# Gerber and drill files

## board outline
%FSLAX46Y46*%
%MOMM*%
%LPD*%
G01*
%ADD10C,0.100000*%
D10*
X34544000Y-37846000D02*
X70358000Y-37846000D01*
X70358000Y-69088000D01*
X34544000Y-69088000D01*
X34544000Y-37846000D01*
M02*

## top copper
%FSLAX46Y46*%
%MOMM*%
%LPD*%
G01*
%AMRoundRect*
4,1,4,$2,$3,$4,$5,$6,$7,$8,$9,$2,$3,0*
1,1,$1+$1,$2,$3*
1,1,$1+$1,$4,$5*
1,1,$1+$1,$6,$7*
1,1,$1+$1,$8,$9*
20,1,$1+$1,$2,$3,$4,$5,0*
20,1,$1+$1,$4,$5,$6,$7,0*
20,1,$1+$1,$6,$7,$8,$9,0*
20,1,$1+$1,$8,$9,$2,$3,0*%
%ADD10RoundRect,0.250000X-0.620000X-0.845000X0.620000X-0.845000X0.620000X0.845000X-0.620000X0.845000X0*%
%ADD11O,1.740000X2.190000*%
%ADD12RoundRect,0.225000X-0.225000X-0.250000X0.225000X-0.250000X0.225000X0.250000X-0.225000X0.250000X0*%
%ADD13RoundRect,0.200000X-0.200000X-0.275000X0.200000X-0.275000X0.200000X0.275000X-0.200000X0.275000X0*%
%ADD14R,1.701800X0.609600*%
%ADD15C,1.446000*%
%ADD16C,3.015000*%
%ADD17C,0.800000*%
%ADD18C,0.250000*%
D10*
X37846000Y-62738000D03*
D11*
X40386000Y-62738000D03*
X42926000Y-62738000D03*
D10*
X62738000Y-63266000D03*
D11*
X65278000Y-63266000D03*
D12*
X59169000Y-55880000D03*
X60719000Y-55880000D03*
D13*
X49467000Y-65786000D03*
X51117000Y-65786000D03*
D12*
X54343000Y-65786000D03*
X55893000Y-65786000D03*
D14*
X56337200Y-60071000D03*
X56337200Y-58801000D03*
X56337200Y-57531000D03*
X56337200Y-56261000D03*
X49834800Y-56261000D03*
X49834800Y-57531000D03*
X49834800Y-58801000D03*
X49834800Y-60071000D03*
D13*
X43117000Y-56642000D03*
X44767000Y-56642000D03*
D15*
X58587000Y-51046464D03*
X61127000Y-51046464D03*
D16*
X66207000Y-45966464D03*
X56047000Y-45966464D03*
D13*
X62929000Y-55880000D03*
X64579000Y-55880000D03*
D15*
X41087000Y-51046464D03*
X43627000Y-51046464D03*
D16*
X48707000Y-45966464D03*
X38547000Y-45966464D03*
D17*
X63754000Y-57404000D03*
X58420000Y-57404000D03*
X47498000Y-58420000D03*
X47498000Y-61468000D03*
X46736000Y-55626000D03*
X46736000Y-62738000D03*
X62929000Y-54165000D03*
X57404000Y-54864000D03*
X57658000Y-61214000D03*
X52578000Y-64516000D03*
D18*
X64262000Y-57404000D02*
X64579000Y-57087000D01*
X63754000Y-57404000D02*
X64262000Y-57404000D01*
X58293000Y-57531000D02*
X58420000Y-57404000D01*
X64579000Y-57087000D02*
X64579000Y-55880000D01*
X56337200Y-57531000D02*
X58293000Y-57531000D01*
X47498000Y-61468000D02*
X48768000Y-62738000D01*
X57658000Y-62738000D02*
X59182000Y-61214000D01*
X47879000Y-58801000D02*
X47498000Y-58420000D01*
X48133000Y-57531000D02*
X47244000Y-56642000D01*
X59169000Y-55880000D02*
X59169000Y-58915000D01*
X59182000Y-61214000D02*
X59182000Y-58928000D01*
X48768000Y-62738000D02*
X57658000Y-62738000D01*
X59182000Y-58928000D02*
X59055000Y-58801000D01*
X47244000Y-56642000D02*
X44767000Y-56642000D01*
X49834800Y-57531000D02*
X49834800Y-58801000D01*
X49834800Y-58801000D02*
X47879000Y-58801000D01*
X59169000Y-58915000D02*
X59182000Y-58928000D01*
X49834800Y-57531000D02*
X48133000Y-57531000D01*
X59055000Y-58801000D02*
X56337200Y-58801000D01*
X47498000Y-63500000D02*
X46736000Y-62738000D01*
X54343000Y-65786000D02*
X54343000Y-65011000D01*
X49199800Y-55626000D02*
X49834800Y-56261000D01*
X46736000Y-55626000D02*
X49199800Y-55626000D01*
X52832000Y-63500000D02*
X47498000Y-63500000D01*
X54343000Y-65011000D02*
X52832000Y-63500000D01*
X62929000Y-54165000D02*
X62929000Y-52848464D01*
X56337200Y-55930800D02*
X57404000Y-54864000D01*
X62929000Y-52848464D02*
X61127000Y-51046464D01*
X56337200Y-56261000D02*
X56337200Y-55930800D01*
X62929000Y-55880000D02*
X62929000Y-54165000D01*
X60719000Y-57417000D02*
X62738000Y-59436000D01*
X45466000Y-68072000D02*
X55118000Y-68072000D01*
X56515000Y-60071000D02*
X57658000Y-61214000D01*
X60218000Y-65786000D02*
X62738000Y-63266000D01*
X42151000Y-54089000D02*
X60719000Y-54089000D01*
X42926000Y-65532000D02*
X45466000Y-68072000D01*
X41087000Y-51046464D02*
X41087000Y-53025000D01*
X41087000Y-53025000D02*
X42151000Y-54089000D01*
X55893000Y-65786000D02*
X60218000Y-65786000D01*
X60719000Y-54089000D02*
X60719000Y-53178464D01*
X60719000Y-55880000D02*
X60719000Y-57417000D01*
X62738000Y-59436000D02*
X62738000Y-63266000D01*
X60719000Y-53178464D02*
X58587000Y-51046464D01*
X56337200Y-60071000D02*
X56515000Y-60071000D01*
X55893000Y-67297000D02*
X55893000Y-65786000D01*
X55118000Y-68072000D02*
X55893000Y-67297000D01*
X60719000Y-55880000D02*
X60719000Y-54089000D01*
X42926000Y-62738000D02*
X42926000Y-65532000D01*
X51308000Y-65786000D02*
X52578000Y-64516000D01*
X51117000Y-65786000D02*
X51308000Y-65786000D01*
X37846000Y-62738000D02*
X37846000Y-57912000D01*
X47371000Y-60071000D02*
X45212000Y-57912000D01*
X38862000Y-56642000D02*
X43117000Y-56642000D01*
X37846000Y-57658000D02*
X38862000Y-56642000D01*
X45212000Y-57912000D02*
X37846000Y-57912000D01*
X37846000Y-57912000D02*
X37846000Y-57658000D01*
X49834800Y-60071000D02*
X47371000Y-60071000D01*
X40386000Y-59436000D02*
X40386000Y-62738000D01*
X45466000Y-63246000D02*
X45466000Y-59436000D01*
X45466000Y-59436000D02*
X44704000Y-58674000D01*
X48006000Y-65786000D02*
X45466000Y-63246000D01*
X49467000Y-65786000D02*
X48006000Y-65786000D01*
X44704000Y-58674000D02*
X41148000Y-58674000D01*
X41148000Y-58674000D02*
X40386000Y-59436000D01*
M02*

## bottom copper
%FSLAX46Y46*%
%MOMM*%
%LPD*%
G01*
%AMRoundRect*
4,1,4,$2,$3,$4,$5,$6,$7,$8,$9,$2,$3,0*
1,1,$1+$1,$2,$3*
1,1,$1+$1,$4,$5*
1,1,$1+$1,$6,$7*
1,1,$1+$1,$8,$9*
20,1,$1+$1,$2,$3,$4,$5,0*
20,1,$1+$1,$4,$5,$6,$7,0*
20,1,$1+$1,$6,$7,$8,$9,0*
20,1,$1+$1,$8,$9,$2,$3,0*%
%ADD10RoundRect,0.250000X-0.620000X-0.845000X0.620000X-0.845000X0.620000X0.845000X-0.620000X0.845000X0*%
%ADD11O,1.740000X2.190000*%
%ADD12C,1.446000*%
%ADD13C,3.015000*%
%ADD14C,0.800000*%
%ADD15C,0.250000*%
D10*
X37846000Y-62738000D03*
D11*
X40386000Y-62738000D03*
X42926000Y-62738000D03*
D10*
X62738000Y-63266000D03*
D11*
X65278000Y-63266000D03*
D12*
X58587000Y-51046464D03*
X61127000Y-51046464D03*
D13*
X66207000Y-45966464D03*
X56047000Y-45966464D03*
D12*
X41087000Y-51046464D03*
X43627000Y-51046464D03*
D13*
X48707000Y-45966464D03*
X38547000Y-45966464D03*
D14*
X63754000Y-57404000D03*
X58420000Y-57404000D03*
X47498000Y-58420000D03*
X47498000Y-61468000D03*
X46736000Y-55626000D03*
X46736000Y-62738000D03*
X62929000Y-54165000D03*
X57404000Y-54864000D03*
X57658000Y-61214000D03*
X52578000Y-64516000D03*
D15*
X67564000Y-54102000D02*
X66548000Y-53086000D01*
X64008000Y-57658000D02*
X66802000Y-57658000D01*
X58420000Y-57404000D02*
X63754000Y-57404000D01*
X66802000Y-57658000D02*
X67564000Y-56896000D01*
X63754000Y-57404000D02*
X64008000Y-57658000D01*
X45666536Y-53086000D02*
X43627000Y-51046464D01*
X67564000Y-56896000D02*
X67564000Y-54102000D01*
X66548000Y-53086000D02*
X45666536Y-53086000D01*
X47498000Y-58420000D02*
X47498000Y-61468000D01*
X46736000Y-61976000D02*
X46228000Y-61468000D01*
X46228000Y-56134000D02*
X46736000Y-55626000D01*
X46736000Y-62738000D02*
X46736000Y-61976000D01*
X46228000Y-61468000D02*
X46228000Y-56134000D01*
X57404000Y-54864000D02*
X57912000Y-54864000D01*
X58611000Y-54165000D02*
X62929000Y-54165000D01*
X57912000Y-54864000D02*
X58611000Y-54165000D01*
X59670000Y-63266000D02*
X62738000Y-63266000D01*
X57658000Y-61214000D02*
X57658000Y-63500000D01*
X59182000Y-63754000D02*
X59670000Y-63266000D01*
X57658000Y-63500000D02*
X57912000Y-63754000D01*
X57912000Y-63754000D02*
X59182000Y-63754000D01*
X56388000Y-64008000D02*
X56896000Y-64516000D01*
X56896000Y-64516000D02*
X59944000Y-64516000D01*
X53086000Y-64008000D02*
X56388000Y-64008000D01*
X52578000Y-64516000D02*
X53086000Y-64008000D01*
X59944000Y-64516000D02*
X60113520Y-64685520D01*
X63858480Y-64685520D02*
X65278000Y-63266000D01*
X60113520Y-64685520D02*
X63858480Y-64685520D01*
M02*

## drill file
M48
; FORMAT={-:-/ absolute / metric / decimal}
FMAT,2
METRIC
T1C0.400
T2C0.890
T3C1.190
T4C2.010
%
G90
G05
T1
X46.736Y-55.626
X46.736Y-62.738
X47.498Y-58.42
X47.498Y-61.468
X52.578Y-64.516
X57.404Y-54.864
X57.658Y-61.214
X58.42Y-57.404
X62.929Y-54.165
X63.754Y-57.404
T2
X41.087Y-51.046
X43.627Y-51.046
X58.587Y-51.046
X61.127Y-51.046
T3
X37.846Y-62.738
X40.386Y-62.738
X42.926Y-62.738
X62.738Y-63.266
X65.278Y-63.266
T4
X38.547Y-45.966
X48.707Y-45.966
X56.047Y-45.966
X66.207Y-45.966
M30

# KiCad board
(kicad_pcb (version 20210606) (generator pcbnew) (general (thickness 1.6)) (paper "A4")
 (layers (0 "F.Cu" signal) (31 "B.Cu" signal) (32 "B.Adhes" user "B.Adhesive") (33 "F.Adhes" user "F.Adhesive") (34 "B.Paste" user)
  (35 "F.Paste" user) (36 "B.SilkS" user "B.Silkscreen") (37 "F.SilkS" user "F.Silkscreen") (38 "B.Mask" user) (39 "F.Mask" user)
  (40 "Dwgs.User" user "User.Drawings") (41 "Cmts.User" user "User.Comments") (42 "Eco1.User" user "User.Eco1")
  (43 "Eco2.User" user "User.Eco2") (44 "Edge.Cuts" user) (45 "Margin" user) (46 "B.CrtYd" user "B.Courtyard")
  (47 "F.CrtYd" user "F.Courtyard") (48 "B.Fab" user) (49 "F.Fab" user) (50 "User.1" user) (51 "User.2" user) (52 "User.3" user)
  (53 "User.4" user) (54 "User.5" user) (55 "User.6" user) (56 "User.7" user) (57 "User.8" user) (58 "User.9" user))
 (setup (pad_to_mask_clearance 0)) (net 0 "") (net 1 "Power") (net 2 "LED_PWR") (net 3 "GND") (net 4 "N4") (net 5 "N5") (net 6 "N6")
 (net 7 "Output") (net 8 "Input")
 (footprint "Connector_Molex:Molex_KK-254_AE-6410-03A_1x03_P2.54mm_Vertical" (layer "F.Cu") (at 37.846 62.738)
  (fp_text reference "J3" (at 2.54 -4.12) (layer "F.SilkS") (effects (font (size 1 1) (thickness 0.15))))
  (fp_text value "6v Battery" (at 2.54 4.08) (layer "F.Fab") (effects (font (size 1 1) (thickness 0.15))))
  (pad "1" thru_hole roundrect locked (at 0 0) (size 1.74 2.19) (drill 1.19) (layers *.Cu *.Mask) (roundrect_rratio 0.1436781609)
   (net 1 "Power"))
  (pad "2" thru_hole oval locked (at 2.54 0) (size 1.74 2.19) (drill 1.19) (layers *.Cu *.Mask) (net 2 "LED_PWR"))
  (pad "3" thru_hole oval locked (at 5.08 0) (size 1.74 2.19) (drill 1.19) (layers *.Cu *.Mask) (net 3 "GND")))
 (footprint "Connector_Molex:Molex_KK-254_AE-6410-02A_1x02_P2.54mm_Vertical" (layer "F.Cu") (at 62.738 63.266)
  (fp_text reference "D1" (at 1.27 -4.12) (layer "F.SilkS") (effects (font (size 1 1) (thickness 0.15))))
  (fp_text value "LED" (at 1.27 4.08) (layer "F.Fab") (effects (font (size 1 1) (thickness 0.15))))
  (pad "1" thru_hole roundrect locked (at 0 0) (size 1.74 2.19) (drill 1.19) (layers *.Cu *.Mask) (roundrect_rratio 0.1436781609)
   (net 3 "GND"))
  (pad "2" thru_hole oval locked (at 2.54 0) (size 1.74 2.19) (drill 1.19) (layers *.Cu *.Mask) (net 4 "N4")))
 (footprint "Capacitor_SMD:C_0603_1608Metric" (layer "F.Cu") (at 59.944 55.88)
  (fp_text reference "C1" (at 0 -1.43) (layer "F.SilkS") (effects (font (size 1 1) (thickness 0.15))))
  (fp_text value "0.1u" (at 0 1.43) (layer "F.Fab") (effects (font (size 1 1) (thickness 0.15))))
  (pad "1" smd roundrect locked (at -0.775 0) (size 0.9 0.95) (layers "F.Cu" "F.Paste" "F.Mask") (roundrect_rratio 0.25) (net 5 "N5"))
  (pad "2" smd roundrect locked (at 0.775 0) (size 0.9 0.95) (layers "F.Cu" "F.Paste" "F.Mask") (roundrect_rratio 0.25) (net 3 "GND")))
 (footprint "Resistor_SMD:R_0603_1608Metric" (layer "F.Cu") (at 50.292 65.786)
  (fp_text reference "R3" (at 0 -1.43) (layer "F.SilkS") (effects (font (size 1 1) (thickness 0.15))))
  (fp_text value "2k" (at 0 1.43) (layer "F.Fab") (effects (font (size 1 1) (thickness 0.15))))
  (pad "1" smd roundrect locked (at -0.825 0) (size 0.8 0.95) (layers "F.Cu" "F.Paste" "F.Mask") (roundrect_rratio 0.25) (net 2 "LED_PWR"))
  (pad "2" smd roundrect locked (at 0.825 0) (size 0.8 0.95) (layers "F.Cu" "F.Paste" "F.Mask") (roundrect_rratio 0.25) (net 4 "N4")))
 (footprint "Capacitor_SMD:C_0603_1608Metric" (layer "F.Cu") (at 55.118 65.786)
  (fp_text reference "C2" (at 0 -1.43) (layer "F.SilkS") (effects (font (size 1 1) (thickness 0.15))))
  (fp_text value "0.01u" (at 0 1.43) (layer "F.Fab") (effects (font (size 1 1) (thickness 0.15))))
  (pad "1" smd roundrect locked (at -0.775 0) (size 0.9 0.95) (layers "F.Cu" "F.Paste" "F.Mask") (roundrect_rratio 0.25) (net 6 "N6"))
  (pad "2" smd roundrect locked (at 0.775 0) (size 0.9 0.95) (layers "F.Cu" "F.Paste" "F.Mask") (roundrect_rratio 0.25) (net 3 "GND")))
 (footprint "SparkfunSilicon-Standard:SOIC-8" (layer "F.Cu") (at 53.086 58.166 90)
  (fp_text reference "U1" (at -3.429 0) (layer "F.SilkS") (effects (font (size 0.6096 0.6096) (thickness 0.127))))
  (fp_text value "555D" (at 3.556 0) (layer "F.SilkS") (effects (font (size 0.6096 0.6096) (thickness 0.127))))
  (pad "1" smd rect locked (at -1.905 3.2512 90) (size 0.6096 1.7018) (layers "F.Cu" "F.Paste" "F.Mask") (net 3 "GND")
   (solder_mask_margin 0.1016))
  (pad "2" smd rect locked (at -0.635 3.2512 90) (size 0.6096 1.7018) (layers "F.Cu" "F.Paste" "F.Mask") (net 5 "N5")
   (solder_mask_margin 0.1016))
  (pad "3" smd rect locked (at 0.635 3.2512 90) (size 0.6096 1.7018) (layers "F.Cu" "F.Paste" "F.Mask") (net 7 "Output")
   (solder_mask_margin 0.1016))
  (pad "4" smd rect locked (at 1.905 3.2512 90) (size 0.6096 1.7018) (layers "F.Cu" "F.Paste" "F.Mask") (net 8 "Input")
   (solder_mask_margin 0.1016))
  (pad "5" smd rect locked (at 1.905 -3.2512 90) (size 0.6096 1.7018) (layers "F.Cu" "F.Paste" "F.Mask") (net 6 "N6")
   (solder_mask_margin 0.1016))
  (pad "6" smd rect locked (at 0.635 -3.2512 90) (size 0.6096 1.7018) (layers "F.Cu" "F.Paste" "F.Mask") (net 5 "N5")
   (solder_mask_margin 0.1016))
  (pad "7" smd rect locked (at -0.635 -3.2512 90) (size 0.6096 1.7018) (layers "F.Cu" "F.Paste" "F.Mask") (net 5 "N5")
   (solder_mask_margin 0.1016))
  (pad "8" smd rect locked (at -1.905 -3.2512 90) (size 0.6096 1.7018) (layers "F.Cu" "F.Paste" "F.Mask") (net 1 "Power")
   (solder_mask_margin 0.1016)))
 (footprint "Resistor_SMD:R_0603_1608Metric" (layer "F.Cu") (at 43.942 56.642)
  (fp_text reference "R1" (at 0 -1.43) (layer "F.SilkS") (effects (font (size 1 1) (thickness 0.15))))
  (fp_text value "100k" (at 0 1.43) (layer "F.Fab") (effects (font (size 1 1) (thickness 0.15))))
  (pad "1" smd roundrect locked (at -0.825 0) (size 0.8 0.95) (layers "F.Cu" "F.Paste" "F.Mask") (roundrect_rratio 0.25) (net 1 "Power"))
  (pad "2" smd roundrect locked (at 0.825 0) (size 0.8 0.95) (layers "F.Cu" "F.Paste" "F.Mask") (roundrect_rratio 0.25) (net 5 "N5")))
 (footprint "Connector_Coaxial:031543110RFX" (layer "F.Cu") (at 58.587 51.046464)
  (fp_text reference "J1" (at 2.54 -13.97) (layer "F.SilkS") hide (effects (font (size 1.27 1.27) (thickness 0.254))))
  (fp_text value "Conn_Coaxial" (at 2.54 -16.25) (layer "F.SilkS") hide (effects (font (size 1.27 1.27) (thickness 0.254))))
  (pad "1" thru_hole circle locked (at 0 0) (size 1.446 1.446) (drill 0.89) (layers *.Cu *.Mask) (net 3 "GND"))
  (pad "2" thru_hole circle locked (at 2.54 0) (size 1.446 1.446) (drill 0.89) (layers *.Cu *.Mask) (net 8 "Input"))
  (pad "3" thru_hole circle locked (at 7.62 -5.08) (size 3.015 3.015) (drill 2.01) (layers *.Cu *.Mask))
  (pad "4" thru_hole circle locked (at -2.54 -5.08) (size 3.015 3.015) (drill 2.01) (layers *.Cu *.Mask)))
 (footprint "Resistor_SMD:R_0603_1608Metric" (layer "F.Cu") (at 63.754 55.88)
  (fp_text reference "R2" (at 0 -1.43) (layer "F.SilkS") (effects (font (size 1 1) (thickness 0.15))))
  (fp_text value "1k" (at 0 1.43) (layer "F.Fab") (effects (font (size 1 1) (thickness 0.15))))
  (pad "1" smd roundrect locked (at -0.825 0) (size 0.8 0.95) (layers "F.Cu" "F.Paste" "F.Mask") (roundrect_rratio 0.25) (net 8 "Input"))
  (pad "2" smd roundrect locked (at 0.825 0) (size 0.8 0.95) (layers "F.Cu" "F.Paste" "F.Mask") (roundrect_rratio 0.25) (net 7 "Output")))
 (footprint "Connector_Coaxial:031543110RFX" (layer "F.Cu") (at 41.087 51.046464)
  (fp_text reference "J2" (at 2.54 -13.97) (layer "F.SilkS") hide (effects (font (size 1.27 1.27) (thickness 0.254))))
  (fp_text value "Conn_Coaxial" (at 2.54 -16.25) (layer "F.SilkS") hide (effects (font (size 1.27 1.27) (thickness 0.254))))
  (pad "1" thru_hole circle locked (at 0 0) (size 1.446 1.446) (drill 0.89) (layers *.Cu *.Mask) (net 3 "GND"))
  (pad "2" thru_hole circle locked (at 2.54 0) (size 1.446 1.446) (drill 0.89) (layers *.Cu *.Mask) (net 7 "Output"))
  (pad "3" thru_hole circle locked (at 7.62 -5.08) (size 3.015 3.015) (drill 2.01) (layers *.Cu *.Mask))
  (pad "4" thru_hole circle locked (at -2.54 -5.08) (size 3.015 3.015) (drill 2.01) (layers *.Cu *.Mask)))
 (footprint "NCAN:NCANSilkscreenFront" (layer "B.Cu") (at 50.8 57.15 180)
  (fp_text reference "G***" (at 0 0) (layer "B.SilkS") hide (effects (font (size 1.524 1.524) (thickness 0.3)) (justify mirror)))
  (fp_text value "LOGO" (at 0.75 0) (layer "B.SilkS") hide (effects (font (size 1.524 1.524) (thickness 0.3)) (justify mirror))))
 (gr_rect (start 34.544 37.846) (end 70.358 69.088) (layer "Edge.Cuts") (width 0.1) (fill none))
 (segment (start 64.262 57.404) (end 64.579 57.087) (width 0.25) (layer "F.Cu") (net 7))
 (segment (start 63.754 57.404) (end 64.262 57.404) (width 0.25) (layer "F.Cu") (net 7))
 (segment (start 58.293 57.531) (end 58.42 57.404) (width 0.25) (layer "F.Cu") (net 7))
 (segment (start 64.579 57.087) (end 64.579 55.88) (width 0.25) (layer "F.Cu") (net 7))
 (segment (start 56.3372 57.531) (end 58.293 57.531) (width 0.25) (layer "F.Cu") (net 7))
 (via (at 63.754 57.404) (size 0.8) (drill 0.4) (layers "F.Cu" "B.Cu") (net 7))
 (via (at 58.42 57.404) (size 0.8) (drill 0.4) (layers "F.Cu" "B.Cu") (free) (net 7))
 (segment (start 67.564 54.102) (end 66.548 53.086) (width 0.25) (layer "B.Cu") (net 7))
 (segment (start 64.008 57.658) (end 66.802 57.658) (width 0.25) (layer "B.Cu") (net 7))
 (segment (start 58.42 57.404) (end 63.754 57.404) (width 0.25) (layer "B.Cu") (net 7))
 (segment (start 66.802 57.658) (end 67.564 56.896) (width 0.25) (layer "B.Cu") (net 7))
 (segment (start 63.754 57.404) (end 64.008 57.658) (width 0.25) (layer "B.Cu") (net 7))
 (segment (start 45.666536 53.086) (end 43.627 51.046464) (width 0.25) (layer "B.Cu") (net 7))
 (segment (start 67.564 56.896) (end 67.564 54.102) (width 0.25) (layer "B.Cu") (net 7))
 (segment (start 66.548 53.086) (end 45.666536 53.086) (width 0.25) (layer "B.Cu") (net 7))
 (segment (start 47.498 61.468) (end 48.768 62.738) (width 0.25) (layer "F.Cu") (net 5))
 (segment (start 57.658 62.738) (end 59.182 61.214) (width 0.25) (layer "F.Cu") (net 5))
 (segment (start 47.879 58.801) (end 47.498 58.42) (width 0.25) (layer "F.Cu") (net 5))
 (segment (start 48.133 57.531) (end 47.244 56.642) (width 0.25) (layer "F.Cu") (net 5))
 (segment (start 59.169 55.88) (end 59.169 58.915) (width 0.25) (layer "F.Cu") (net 5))
 (segment (start 59.182 61.214) (end 59.182 58.928) (width 0.25) (layer "F.Cu") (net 5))
 (segment (start 48.768 62.738) (end 57.658 62.738) (width 0.25) (layer "F.Cu") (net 5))
 (segment (start 59.182 58.928) (end 59.055 58.801) (width 0.25) (layer "F.Cu") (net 5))
 (segment (start 47.244 56.642) (end 44.767 56.642) (width 0.25) (layer "F.Cu") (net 5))
 (segment (start 49.8348 57.531) (end 49.8348 58.801) (width 0.25) (layer "F.Cu") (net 5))
 (segment (start 49.8348 58.801) (end 47.879 58.801) (width 0.25) (layer "F.Cu") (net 5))
 (segment (start 59.169 58.915) (end 59.182 58.928) (width 0.25) (layer "F.Cu") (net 5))
 (segment (start 49.8348 57.531) (end 48.133 57.531) (width 0.25) (layer "F.Cu") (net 5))
 (segment (start 59.055 58.801) (end 56.3372 58.801) (width 0.25) (layer "F.Cu") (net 5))
 (via (at 47.498 58.42) (size 0.8) (drill 0.4) (layers "F.Cu" "B.Cu") (free) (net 5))
 (via (at 47.498 61.468) (size 0.8) (drill 0.4) (layers "F.Cu" "B.Cu") (free) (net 5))
 (segment (start 47.498 58.42) (end 47.498 61.468) (width 0.25) (layer "B.Cu") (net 5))
 (segment (start 47.498 63.5) (end 46.736 62.738) (width 0.25) (layer "F.Cu") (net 6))
 (segment (start 54.343 65.786) (end 54.343 65.011) (width 0.25) (layer "F.Cu") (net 6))
 (segment (start 49.1998 55.626) (end 49.8348 56.261) (width 0.25) (layer "F.Cu") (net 6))
 (segment (start 46.736 55.626) (end 49.1998 55.626) (width 0.25) (layer "F.Cu") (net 6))
 (segment (start 52.832 63.5) (end 47.498 63.5) (width 0.25) (layer "F.Cu") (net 6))
 (segment (start 54.343 65.011) (end 52.832 63.5) (width 0.25) (layer "F.Cu") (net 6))
 (via (at 46.736 55.626) (size 0.8) (drill 0.4) (layers "F.Cu" "B.Cu") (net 6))
 (via (at 46.736 62.738) (size 0.8) (drill 0.4) (layers "F.Cu" "B.Cu") (free) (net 6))
 (segment (start 46.736 61.976) (end 46.228 61.468) (width 0.25) (layer "B.Cu") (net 6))
 (segment (start 46.228 56.134) (end 46.736 55.626) (width 0.25) (layer "B.Cu") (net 6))
 (segment (start 46.736 62.738) (end 46.736 61.976) (width 0.25) (layer "B.Cu") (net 6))
 (segment (start 46.228 61.468) (end 46.228 56.134) (width 0.25) (layer "B.Cu") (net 6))
 (segment (start 62.929 54.165) (end 62.929 52.848464) (width 0.25) (layer "F.Cu") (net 8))
 (segment (start 56.3372 55.9308) (end 57.404 54.864) (width 0.25) (layer "F.Cu") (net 8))
 (segment (start 62.929 52.848464) (end 61.127 51.046464) (width 0.25) (layer "F.Cu") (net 8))
 (segment (start 56.3372 56.261) (end 56.3372 55.9308) (width 0.25) (layer "F.Cu") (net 8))
 (segment (start 62.929 55.88) (end 62.929 54.165) (width 0.25) (layer "F.Cu") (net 8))
 (via (at 62.929 54.165) (size 0.8) (drill 0.4) (layers "F.Cu" "B.Cu") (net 8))
 (via (at 57.404 54.864) (size 0.8) (drill 0.4) (layers "F.Cu" "B.Cu") (free) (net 8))
 (segment (start 57.404 54.864) (end 57.912 54.864) (width 0.25) (layer "B.Cu") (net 8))
 (segment (start 58.611 54.165) (end 62.929 54.165) (width 0.25) (layer "B.Cu") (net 8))
 (segment (start 57.912 54.864) (end 58.611 54.165) (width 0.25) (layer "B.Cu") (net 8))
 (segment (start 60.719 57.417) (end 62.738 59.436) (width 0.25) (layer "F.Cu") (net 3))
 (segment (start 45.466 68.072) (end 55.118 68.072) (width 0.25) (layer "F.Cu") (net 3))
 (segment (start 56.515 60.071) (end 57.658 61.214) (width 0.25) (layer "F.Cu") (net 3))
 (segment (start 60.218 65.786) (end 62.738 63.266) (width 0.25) (layer "F.Cu") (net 3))
 (segment (start 42.151 54.089) (end 60.719 54.089) (width 0.25) (layer "F.Cu") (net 3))
 (segment (start 42.926 65.532) (end 45.466 68.072) (width 0.25) (layer "F.Cu") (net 3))
 (segment (start 41.087 51.046464) (end 41.087 53.025) (width 0.25) (layer "F.Cu") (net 3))
 (segment (start 41.087 53.025) (end 42.151 54.089) (width 0.25) (layer "F.Cu") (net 3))
 (segment (start 55.893 65.786) (end 60.218 65.786) (width 0.25) (layer "F.Cu") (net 3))
 (segment (start 60.719 54.089) (end 60.719 53.178464) (width 0.25) (layer "F.Cu") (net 3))
 (segment (start 60.719 55.88) (end 60.719 57.417) (width 0.25) (layer "F.Cu") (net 3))
 (segment (start 62.738 59.436) (end 62.738 63.266) (width 0.25) (layer "F.Cu") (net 3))
 (segment (start 60.719 53.178464) (end 58.587 51.046464) (width 0.25) (layer "F.Cu") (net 3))
 (segment (start 56.3372 60.071) (end 56.515 60.071) (width 0.25) (layer "F.Cu") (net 3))
 (segment (start 55.893 67.297) (end 55.893 65.786) (width 0.25) (layer "F.Cu") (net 3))
 (segment (start 55.118 68.072) (end 55.893 67.297) (width 0.25) (layer "F.Cu") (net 3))
 (segment (start 60.719 55.88) (end 60.719 54.089) (width 0.25) (layer "F.Cu") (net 3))
 (segment (start 42.926 62.738) (end 42.926 65.532) (width 0.25) (layer "F.Cu") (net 3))
 (via (at 57.658 61.214) (size 0.8) (drill 0.4) (layers "F.Cu" "B.Cu") (free) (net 3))
 (segment (start 59.67 63.266) (end 62.738 63.266) (width 0.25) (layer "B.Cu") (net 3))
 (segment (start 57.658 61.214) (end 57.658 63.5) (width 0.25) (layer "B.Cu") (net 3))
 (segment (start 59.182 63.754) (end 59.67 63.266) (width 0.25) (layer "B.Cu") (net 3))
 (segment (start 57.658 63.5) (end 57.912 63.754) (width 0.25) (layer "B.Cu") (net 3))
 (segment (start 57.912 63.754) (end 59.182 63.754) (width 0.25) (layer "B.Cu") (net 3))
 (segment (start 51.308 65.786) (end 52.578 64.516) (width 0.25) (layer "F.Cu") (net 4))
 (segment (start 51.117 65.786) (end 51.308 65.786) (width 0.25) (layer "F.Cu") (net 4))
 (via (at 52.578 64.516) (size 0.8) (drill 0.4) (layers "F.Cu" "B.Cu") (free) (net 4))
 (segment (start 56.388 64.008) (end 56.896 64.516) (width 0.25) (layer "B.Cu") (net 4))
 (segment (start 56.896 64.516) (end 59.944 64.516) (width 0.25) (layer "B.Cu") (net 4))
 (segment (start 53.086 64.008) (end 56.388 64.008) (width 0.25) (layer "B.Cu") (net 4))
 (segment (start 52.578 64.516) (end 53.086 64.008) (width 0.25) (layer "B.Cu") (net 4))
 (segment (start 59.944 64.516) (end 60.11352 64.68552) (width 0.25) (layer "B.Cu") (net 4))
 (segment (start 63.85848 64.68552) (end 65.278 63.266) (width 0.25) (layer "B.Cu") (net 4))
 (segment (start 60.11352 64.68552) (end 63.85848 64.68552) (width 0.25) (layer "B.Cu") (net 4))
 (segment (start 37.846 62.738) (end 37.846 57.912) (width 0.25) (layer "F.Cu") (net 1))
 (segment (start 47.371 60.071) (end 45.212 57.912) (width 0.25) (layer "F.Cu") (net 1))
 (segment (start 38.862 56.642) (end 43.117 56.642) (width 0.25) (layer "F.Cu") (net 1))
 (segment (start 37.846 57.658) (end 38.862 56.642) (width 0.25) (layer "F.Cu") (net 1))
 (segment (start 45.212 57.912) (end 37.846 57.912) (width 0.25) (layer "F.Cu") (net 1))
 (segment (start 37.846 57.912) (end 37.846 57.658) (width 0.25) (layer "F.Cu") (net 1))
 (segment (start 49.8348 60.071) (end 47.371 60.071) (width 0.25) (layer "F.Cu") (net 1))
 (segment (start 40.386 59.436) (end 40.386 62.738) (width 0.25) (layer "F.Cu") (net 2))
 (segment (start 45.466 63.246) (end 45.466 59.436) (width 0.25) (layer "F.Cu") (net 2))
 (segment (start 45.466 59.436) (end 44.704 58.674) (width 0.25) (layer "F.Cu") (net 2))
 (segment (start 48.006 65.786) (end 45.466 63.246) (width 0.25) (layer "F.Cu") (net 2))
 (segment (start 49.467 65.786) (end 48.006 65.786) (width 0.25) (layer "F.Cu") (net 2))
 (segment (start 44.704 58.674) (end 41.148 58.674) (width 0.25) (layer "F.Cu") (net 2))
 (segment (start 41.148 58.674) (end 40.386 59.436) (width 0.25) (layer "F.Cu") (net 2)))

